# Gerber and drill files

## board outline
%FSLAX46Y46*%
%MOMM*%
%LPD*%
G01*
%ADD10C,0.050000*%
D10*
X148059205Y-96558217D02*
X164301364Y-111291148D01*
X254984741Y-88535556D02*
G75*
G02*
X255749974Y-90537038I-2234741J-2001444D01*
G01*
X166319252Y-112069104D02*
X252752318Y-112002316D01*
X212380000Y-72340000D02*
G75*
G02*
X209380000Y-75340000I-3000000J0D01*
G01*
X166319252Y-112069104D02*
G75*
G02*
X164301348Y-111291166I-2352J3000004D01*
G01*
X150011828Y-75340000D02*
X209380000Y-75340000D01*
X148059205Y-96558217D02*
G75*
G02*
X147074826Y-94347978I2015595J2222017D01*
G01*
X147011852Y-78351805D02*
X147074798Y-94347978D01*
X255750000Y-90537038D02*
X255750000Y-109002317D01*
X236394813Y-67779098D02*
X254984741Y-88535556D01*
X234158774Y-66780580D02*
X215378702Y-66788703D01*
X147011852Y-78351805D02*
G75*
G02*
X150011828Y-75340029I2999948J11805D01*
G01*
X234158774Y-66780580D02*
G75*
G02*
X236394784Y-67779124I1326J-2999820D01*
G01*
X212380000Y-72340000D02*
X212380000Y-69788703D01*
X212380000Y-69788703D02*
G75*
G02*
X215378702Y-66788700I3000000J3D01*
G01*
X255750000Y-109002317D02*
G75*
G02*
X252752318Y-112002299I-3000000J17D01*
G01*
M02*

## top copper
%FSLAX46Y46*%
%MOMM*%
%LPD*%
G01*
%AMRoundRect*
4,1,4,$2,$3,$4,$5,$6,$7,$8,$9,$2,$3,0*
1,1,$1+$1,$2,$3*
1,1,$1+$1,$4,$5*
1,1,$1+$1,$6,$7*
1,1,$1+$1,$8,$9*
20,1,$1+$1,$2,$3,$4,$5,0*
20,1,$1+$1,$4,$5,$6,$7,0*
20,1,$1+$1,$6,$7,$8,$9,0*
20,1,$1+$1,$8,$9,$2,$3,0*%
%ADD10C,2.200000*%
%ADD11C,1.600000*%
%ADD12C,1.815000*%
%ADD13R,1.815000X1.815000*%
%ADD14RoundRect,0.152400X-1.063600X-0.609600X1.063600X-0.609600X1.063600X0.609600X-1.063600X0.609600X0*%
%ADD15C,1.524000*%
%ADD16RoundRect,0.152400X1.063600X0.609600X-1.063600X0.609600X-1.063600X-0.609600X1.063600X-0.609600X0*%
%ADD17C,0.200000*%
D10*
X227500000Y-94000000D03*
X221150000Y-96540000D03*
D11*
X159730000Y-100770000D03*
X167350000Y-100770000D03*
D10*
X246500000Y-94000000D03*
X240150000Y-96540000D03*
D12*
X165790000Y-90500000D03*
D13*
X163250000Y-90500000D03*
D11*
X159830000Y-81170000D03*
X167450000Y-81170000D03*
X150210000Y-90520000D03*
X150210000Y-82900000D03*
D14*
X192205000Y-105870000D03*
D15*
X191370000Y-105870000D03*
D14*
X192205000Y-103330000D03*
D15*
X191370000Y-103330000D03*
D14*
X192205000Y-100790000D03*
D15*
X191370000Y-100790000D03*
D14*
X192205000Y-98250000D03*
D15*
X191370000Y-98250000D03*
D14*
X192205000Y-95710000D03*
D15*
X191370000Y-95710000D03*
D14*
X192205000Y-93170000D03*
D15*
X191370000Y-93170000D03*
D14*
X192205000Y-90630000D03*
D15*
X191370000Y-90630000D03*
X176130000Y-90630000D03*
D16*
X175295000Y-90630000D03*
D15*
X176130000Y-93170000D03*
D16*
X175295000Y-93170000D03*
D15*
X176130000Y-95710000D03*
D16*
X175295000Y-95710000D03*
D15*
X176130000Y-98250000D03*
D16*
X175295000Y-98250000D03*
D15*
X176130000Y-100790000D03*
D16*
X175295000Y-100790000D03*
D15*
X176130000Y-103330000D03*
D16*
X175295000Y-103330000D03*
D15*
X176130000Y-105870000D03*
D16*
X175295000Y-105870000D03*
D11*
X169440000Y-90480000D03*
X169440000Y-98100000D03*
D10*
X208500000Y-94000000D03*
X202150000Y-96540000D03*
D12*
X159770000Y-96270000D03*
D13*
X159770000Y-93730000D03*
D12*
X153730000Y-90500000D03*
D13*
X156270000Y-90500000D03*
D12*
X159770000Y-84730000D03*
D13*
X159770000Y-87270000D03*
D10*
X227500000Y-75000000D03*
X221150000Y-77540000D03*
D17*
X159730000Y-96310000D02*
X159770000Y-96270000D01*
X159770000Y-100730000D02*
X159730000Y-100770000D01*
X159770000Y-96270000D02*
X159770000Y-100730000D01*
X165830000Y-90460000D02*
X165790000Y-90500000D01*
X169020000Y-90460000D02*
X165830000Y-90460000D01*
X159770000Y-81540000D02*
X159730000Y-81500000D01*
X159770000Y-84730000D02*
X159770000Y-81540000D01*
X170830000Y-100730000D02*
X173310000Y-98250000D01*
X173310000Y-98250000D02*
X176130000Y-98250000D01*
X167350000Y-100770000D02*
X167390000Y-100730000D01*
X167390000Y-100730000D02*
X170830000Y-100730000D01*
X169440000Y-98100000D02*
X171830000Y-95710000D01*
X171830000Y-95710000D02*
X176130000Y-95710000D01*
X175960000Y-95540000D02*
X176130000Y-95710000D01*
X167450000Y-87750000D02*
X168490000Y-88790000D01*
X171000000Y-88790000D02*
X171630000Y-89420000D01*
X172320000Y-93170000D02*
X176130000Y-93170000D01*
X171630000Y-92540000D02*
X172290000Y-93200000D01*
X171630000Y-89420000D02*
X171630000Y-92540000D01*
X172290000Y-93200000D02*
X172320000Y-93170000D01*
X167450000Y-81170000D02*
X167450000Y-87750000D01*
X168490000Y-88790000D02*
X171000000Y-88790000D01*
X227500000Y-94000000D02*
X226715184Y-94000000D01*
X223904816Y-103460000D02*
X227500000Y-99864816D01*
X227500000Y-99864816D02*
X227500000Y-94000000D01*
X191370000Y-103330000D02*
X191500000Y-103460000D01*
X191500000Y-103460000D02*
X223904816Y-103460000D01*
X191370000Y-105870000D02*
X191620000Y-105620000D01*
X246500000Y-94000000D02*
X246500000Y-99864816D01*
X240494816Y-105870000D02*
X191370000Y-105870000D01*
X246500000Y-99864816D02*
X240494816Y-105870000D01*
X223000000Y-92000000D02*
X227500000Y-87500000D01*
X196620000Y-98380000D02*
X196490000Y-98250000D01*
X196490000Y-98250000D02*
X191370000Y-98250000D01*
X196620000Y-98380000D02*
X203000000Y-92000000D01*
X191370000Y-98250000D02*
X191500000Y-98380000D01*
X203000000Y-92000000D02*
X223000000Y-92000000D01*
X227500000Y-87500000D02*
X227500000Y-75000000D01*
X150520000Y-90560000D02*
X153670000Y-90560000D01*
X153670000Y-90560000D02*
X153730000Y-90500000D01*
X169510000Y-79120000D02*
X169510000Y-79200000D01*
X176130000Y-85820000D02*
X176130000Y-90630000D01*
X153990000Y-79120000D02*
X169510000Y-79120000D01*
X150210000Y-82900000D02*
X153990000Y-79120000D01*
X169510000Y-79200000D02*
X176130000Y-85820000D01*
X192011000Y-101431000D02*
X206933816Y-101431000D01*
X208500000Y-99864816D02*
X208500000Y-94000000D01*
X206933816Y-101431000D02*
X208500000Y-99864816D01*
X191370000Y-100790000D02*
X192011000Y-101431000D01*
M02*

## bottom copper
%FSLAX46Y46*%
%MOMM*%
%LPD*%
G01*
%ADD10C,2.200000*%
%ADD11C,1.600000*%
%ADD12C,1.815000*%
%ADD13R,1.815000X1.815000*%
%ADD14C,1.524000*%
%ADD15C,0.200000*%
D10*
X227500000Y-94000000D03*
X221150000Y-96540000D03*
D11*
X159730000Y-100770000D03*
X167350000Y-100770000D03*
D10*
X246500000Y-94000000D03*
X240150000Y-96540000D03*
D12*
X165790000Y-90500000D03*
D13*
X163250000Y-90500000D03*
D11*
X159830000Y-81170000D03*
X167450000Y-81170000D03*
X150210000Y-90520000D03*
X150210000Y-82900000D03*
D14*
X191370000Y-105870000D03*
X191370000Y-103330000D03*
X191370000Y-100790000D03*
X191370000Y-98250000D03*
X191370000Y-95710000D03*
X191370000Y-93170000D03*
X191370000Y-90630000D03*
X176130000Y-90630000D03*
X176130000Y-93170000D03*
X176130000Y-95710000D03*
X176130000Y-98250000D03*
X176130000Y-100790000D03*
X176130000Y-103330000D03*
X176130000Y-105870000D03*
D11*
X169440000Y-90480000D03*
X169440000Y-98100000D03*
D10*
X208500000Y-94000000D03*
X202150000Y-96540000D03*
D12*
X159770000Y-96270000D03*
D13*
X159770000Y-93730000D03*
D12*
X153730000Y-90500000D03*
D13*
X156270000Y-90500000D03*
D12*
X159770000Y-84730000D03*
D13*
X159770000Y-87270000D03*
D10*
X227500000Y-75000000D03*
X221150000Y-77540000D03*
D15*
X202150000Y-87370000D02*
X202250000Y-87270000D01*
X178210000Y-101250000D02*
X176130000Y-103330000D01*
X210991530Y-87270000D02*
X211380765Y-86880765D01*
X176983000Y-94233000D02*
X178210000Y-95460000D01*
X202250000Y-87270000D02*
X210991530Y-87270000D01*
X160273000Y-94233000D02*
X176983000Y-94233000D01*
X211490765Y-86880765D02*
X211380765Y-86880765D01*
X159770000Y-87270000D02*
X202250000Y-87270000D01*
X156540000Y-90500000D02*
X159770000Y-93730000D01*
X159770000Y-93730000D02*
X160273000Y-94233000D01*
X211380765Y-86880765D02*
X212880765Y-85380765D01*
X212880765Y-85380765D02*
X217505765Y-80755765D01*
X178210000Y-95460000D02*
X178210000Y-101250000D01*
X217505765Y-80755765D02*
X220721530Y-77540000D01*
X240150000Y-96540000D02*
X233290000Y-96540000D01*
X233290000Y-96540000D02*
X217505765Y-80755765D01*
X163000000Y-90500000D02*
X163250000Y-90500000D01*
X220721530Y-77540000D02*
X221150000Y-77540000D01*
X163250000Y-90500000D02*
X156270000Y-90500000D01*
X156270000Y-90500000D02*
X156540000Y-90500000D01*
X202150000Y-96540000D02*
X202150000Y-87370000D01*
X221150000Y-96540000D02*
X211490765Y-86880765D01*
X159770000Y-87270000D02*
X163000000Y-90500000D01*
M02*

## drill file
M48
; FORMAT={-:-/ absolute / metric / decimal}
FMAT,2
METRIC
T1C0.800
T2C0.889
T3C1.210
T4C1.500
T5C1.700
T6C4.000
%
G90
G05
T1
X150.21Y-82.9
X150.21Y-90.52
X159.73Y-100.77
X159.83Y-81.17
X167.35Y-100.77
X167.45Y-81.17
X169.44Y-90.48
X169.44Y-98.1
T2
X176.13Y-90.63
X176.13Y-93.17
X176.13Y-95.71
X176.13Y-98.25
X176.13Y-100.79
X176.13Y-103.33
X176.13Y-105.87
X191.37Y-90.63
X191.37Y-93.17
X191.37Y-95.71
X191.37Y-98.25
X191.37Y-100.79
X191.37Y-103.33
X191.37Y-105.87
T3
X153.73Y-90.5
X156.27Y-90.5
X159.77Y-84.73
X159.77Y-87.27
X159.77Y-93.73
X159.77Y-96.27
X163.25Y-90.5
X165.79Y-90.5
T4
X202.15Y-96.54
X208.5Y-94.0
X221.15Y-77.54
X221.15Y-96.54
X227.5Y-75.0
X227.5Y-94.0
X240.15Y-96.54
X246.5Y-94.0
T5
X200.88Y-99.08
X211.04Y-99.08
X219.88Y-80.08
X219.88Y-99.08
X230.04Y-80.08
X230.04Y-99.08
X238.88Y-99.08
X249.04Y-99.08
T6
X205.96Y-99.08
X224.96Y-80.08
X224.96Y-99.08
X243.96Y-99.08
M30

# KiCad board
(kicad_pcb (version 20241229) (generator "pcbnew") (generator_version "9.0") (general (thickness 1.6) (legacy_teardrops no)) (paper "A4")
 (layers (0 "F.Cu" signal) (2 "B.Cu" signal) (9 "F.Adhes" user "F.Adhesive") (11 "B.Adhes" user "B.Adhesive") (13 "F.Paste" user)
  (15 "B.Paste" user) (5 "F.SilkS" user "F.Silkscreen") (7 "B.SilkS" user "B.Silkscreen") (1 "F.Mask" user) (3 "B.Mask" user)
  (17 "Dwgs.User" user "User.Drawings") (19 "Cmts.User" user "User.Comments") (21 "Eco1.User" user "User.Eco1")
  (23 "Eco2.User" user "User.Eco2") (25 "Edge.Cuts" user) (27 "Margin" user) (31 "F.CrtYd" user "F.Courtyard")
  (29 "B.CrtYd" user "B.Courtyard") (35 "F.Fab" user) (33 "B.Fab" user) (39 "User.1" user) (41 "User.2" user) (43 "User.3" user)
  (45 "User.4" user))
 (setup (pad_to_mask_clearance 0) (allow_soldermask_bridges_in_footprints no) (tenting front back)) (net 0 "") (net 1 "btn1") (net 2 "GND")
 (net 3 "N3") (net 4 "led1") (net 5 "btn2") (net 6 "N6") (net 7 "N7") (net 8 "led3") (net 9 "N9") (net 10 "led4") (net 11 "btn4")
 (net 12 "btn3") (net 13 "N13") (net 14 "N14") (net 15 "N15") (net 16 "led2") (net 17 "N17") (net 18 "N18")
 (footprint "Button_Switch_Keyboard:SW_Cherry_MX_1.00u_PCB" (layer "F.Cu") (at 227.5 94)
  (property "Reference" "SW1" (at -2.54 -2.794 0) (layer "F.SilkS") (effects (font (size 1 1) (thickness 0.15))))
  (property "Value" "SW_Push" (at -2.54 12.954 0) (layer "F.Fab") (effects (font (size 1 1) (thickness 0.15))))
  (pad "" np_thru_hole circle (at -7.62 5.08) (size 1.7 1.7) (drill 1.7) (layers "*.Cu" "*.Mask"))
  (pad "" np_thru_hole circle (at -2.54 5.08) (size 4 4) (drill 4) (layers "*.Cu" "*.Mask"))
  (pad "" np_thru_hole circle (at 2.54 5.08) (size 1.7 1.7) (drill 1.7) (layers "*.Cu" "*.Mask"))
  (pad "1" thru_hole circle (at 0 0) (size 2.2 2.2) (drill 1.5) (layers "*.Cu" "*.Mask") (remove_unused_layers no) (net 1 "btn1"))
  (pad "2" thru_hole circle (at -6.35 2.54) (size 2.2 2.2) (drill 1.5) (layers "*.Cu" "*.Mask") (remove_unused_layers no) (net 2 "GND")))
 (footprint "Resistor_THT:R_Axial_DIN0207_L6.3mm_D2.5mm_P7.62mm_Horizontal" (layer "F.Cu") (at 159.73 100.77)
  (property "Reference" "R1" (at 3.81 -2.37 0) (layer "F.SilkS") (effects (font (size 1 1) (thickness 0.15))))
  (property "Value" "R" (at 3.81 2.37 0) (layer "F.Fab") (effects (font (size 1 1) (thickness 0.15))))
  (pad "1" thru_hole circle (at 0 0) (size 1.6 1.6) (drill 0.8) (layers "*.Cu" "*.Mask") (remove_unused_layers no) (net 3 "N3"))
  (pad "2" thru_hole circle (at 7.62 0) (size 1.6 1.6) (drill 0.8) (layers "*.Cu" "*.Mask") (remove_unused_layers no) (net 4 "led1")))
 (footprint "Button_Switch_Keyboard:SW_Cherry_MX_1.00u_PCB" (layer "F.Cu") (at 246.5 94)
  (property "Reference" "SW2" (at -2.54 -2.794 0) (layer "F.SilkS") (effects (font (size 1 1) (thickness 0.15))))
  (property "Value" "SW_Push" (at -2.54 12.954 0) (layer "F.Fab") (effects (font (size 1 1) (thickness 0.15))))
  (pad "" np_thru_hole circle (at -7.62 5.08) (size 1.7 1.7) (drill 1.7) (layers "*.Cu" "*.Mask"))
  (pad "" np_thru_hole circle (at -2.54 5.08) (size 4 4) (drill 4) (layers "*.Cu" "*.Mask"))
  (pad "" np_thru_hole circle (at 2.54 5.08) (size 1.7 1.7) (drill 1.7) (layers "*.Cu" "*.Mask"))
  (pad "1" thru_hole circle (at 0 0) (size 2.2 2.2) (drill 1.5) (layers "*.Cu" "*.Mask") (remove_unused_layers no) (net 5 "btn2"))
  (pad "2" thru_hole circle (at -6.35 2.54) (size 2.2 2.2) (drill 1.5) (layers "*.Cu" "*.Mask") (remove_unused_layers no) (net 2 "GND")))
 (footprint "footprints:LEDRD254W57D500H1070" (layer "F.Cu") (at 164.52 90.5)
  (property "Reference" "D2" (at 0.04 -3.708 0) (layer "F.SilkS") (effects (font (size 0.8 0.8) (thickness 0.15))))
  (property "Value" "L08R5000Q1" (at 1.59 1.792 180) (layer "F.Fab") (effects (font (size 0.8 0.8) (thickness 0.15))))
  (pad "A" thru_hole circle (at 1.27 0) (size 1.815 1.815) (drill 1.21) (layers "*.Cu" "*.Mask") (remove_unused_layers no) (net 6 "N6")
   (solder_mask_margin 0.102))
  (pad "C" thru_hole rect (at -1.27 0) (size 1.815 1.815) (drill 1.21) (layers "*.Cu" "*.Mask") (remove_unused_layers no) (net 2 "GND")
   (solder_mask_margin 0.102)))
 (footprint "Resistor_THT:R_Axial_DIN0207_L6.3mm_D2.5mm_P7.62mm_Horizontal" (layer "F.Cu") (at 159.83 81.17)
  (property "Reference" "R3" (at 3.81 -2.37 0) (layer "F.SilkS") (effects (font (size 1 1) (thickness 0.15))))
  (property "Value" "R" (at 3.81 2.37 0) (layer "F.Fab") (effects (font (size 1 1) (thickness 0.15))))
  (pad "1" thru_hole circle (at 0 0) (size 1.6 1.6) (drill 0.8) (layers "*.Cu" "*.Mask") (remove_unused_layers no) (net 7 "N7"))
  (pad "2" thru_hole circle (at 7.62 0) (size 1.6 1.6) (drill 0.8) (layers "*.Cu" "*.Mask") (remove_unused_layers no) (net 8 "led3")))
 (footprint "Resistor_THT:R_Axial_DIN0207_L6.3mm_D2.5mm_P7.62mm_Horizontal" (layer "F.Cu") (at 150.21 90.52 90)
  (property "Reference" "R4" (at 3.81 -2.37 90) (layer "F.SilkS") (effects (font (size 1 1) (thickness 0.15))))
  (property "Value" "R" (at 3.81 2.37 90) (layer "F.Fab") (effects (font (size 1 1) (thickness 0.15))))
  (pad "1" thru_hole circle (at 0 0 90) (size 1.6 1.6) (drill 0.8) (layers "*.Cu" "*.Mask") (remove_unused_layers no) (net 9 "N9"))
  (pad "2" thru_hole circle (at 7.62 0 90) (size 1.6 1.6) (drill 0.8) (layers "*.Cu" "*.Mask") (remove_unused_layers no) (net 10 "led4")))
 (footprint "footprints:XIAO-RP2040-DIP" (layer "F.Cu") (at 183.75 98.25 -90)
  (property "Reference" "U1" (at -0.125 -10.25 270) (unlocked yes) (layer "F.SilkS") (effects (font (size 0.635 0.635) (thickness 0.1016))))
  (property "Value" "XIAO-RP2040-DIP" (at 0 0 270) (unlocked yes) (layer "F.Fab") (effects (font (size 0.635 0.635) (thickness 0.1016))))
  (pad "1" smd roundrect (at 7.62 -8.455) (size 2.432 1.524) (layers "F.Cu" "F.Mask") (roundrect_rratio 0.1) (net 5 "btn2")
   (thermal_bridge_angle 45))
  (pad "1" thru_hole circle (at 7.62 -7.62) (size 1.524 1.524) (drill 0.889) (layers "*.Cu" "*.Mask") (remove_unused_layers no)
   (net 5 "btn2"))
  (pad "2" smd roundrect (at 5.08 -8.455) (size 2.432 1.524) (layers "F.Cu" "F.Mask") (roundrect_rratio 0.1) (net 1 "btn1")
   (thermal_bridge_angle 45))
  (pad "2" thru_hole circle (at 5.08 -7.62) (size 1.524 1.524) (drill 0.889) (layers "*.Cu" "*.Mask") (remove_unused_layers no)
   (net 1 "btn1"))
  (pad "3" smd roundrect (at 2.54 -8.455) (size 2.432 1.524) (layers "F.Cu" "F.Mask") (roundrect_rratio 0.1) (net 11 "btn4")
   (thermal_bridge_angle 45))
  (pad "3" thru_hole circle (at 2.54 -7.62) (size 1.524 1.524) (drill 0.889) (layers "*.Cu" "*.Mask") (remove_unused_layers no)
   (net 11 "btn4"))
  (pad "4" smd roundrect (at 0 -8.455) (size 2.432 1.524) (layers "F.Cu" "F.Mask") (roundrect_rratio 0.1) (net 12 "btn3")
   (thermal_bridge_angle 45))
  (pad "4" thru_hole circle (at 0 -7.62) (size 1.524 1.524) (drill 0.889) (layers "*.Cu" "*.Mask") (remove_unused_layers no) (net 12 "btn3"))
  (pad "5" smd roundrect (at -2.54 -8.455) (size 2.432 1.524) (layers "F.Cu" "F.Mask") (roundrect_rratio 0.1) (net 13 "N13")
   (thermal_bridge_angle 45))
  (pad "5" thru_hole circle (at -2.54 -7.62) (size 1.524 1.524) (drill 0.889) (layers "*.Cu" "*.Mask") (remove_unused_layers no)
   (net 13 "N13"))
  (pad "6" smd roundrect (at -5.08 -8.455) (size 2.432 1.524) (layers "F.Cu" "F.Mask") (roundrect_rratio 0.1) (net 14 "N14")
   (thermal_bridge_angle 45))
  (pad "6" thru_hole circle (at -5.08 -7.62) (size 1.524 1.524) (drill 0.889) (layers "*.Cu" "*.Mask") (remove_unused_layers no)
   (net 14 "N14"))
  (pad "7" smd roundrect (at -7.62 -8.455) (size 2.432 1.524) (layers "F.Cu" "F.Mask") (roundrect_rratio 0.1) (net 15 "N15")
   (thermal_bridge_angle 45))
  (pad "7" thru_hole circle (at -7.62 -7.62) (size 1.524 1.524) (drill 0.889) (layers "*.Cu" "*.Mask") (remove_unused_layers no)
   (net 15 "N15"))
  (pad "8" thru_hole circle (at -7.62 7.62 180) (size 1.524 1.524) (drill 0.889) (layers "*.Cu" "*.Mask") (remove_unused_layers no)
   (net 10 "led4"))
  (pad "8" smd roundrect (at -7.62 8.455 180) (size 2.432 1.524) (layers "F.Cu" "F.Mask") (roundrect_rratio 0.1) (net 10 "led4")
   (thermal_bridge_angle 45))
  (pad "9" thru_hole circle (at -5.08 7.62 180) (size 1.524 1.524) (drill 0.889) (layers "*.Cu" "*.Mask") (remove_unused_layers no)
   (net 8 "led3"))
  (pad "9" smd roundrect (at -5.08 8.455 180) (size 2.432 1.524) (layers "F.Cu" "F.Mask") (roundrect_rratio 0.1) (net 8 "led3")
   (thermal_bridge_angle 45))
  (pad "10" thru_hole circle (at -2.54 7.62 180) (size 1.524 1.524) (drill 0.889) (layers "*.Cu" "*.Mask") (remove_unused_layers no)
   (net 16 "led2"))
  (pad "10" smd roundrect (at -2.54 8.455 180) (size 2.432 1.524) (layers "F.Cu" "F.Mask") (roundrect_rratio 0.1) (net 16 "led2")
   (thermal_bridge_angle 45))
  (pad "11" thru_hole circle (at 0 7.62 180) (size 1.524 1.524) (drill 0.889) (layers "*.Cu" "*.Mask") (remove_unused_layers no)
   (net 4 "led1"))
  (pad "11" smd roundrect (at 0 8.455 180) (size 2.432 1.524) (layers "F.Cu" "F.Mask") (roundrect_rratio 0.1) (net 4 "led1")
   (thermal_bridge_angle 45))
  (pad "12" thru_hole circle (at 2.54 7.62 180) (size 1.524 1.524) (drill 0.889) (layers "*.Cu" "*.Mask") (remove_unused_layers no)
   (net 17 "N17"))
  (pad "12" smd roundrect (at 2.54 8.455 180) (size 2.432 1.524) (layers "F.Cu" "F.Mask") (roundrect_rratio 0.1) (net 17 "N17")
   (thermal_bridge_angle 45))
  (pad "13" thru_hole circle (at 5.08 7.62 180) (size 1.524 1.524) (drill 0.889) (layers "*.Cu" "*.Mask") (remove_unused_layers no)
   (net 2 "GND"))
  (pad "13" smd roundrect (at 5.08 8.455 180) (size 2.432 1.524) (layers "F.Cu" "F.Mask") (roundrect_rratio 0.1) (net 2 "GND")
   (thermal_bridge_angle 45))
  (pad "14" thru_hole circle (at 7.62 7.62 180) (size 1.524 1.524) (drill 0.889) (layers "*.Cu" "*.Mask") (remove_unused_layers no)
   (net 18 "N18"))
  (pad "14" smd roundrect (at 7.62 8.455 180) (size 2.432 1.524) (layers "F.Cu" "F.Mask") (roundrect_rratio 0.1) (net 18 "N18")
   (thermal_bridge_angle 45)))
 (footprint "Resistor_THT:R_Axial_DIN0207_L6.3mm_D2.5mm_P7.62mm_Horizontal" (layer "F.Cu") (at 169.44 90.48 -90)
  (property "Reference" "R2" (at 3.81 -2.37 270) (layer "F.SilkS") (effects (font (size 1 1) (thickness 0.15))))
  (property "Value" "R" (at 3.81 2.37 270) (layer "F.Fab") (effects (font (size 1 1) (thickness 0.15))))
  (pad "1" thru_hole circle (at 0 0 270) (size 1.6 1.6) (drill 0.8) (layers "*.Cu" "*.Mask") (remove_unused_layers no) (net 6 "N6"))
  (pad "2" thru_hole circle (at 7.62 0 270) (size 1.6 1.6) (drill 0.8) (layers "*.Cu" "*.Mask") (remove_unused_layers no) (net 16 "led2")))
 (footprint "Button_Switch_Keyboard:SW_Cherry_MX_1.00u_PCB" (layer "F.Cu") (at 208.5 94)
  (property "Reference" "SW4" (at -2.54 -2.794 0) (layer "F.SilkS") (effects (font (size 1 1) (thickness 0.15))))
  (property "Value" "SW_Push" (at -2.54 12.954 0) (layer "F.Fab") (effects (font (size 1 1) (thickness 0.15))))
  (pad "" np_thru_hole circle (at -7.62 5.08) (size 1.7 1.7) (drill 1.7) (layers "*.Cu" "*.Mask"))
  (pad "" np_thru_hole circle (at -2.54 5.08) (size 4 4) (drill 4) (layers "*.Cu" "*.Mask"))
  (pad "" np_thru_hole circle (at 2.54 5.08) (size 1.7 1.7) (drill 1.7) (layers "*.Cu" "*.Mask"))
  (pad "1" thru_hole circle (at 0 0) (size 2.2 2.2) (drill 1.5) (layers "*.Cu" "*.Mask") (remove_unused_layers no) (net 11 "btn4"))
  (pad "2" thru_hole circle (at -6.35 2.54) (size 2.2 2.2) (drill 1.5) (layers "*.Cu" "*.Mask") (remove_unused_layers no) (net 2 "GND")))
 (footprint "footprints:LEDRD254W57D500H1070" (layer "F.Cu") (at 159.77 95 -90)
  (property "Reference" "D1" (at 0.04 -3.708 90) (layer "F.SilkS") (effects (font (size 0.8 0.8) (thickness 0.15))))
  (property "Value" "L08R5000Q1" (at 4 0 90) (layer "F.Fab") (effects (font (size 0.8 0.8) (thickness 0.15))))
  (pad "A" thru_hole circle (at 1.27 0 270) (size 1.815 1.815) (drill 1.21) (layers "*.Cu" "*.Mask") (remove_unused_layers no) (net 3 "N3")
   (solder_mask_margin 0.102))
  (pad "C" thru_hole rect (at -1.27 0 270) (size 1.815 1.815) (drill 1.21) (layers "*.Cu" "*.Mask") (remove_unused_layers no) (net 2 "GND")
   (solder_mask_margin 0.102)))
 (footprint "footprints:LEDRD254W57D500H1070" (layer "F.Cu") (at 155 90.5 180)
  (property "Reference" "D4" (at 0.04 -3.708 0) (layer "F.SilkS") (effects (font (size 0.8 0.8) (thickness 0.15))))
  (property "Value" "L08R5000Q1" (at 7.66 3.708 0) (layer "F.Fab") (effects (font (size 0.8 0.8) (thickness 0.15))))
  (pad "A" thru_hole circle (at 1.27 0 180) (size 1.815 1.815) (drill 1.21) (layers "*.Cu" "*.Mask") (remove_unused_layers no) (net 9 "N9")
   (solder_mask_margin 0.102))
  (pad "C" thru_hole rect (at -1.27 0 180) (size 1.815 1.815) (drill 1.21) (layers "*.Cu" "*.Mask") (remove_unused_layers no) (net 2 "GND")
   (solder_mask_margin 0.102)))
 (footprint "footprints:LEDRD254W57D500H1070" (layer "F.Cu") (at 159.77 86 90)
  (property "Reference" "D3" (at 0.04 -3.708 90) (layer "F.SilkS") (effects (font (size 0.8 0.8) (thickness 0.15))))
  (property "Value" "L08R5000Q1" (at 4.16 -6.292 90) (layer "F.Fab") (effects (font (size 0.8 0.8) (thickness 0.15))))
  (pad "A" thru_hole circle (at 1.27 0 90) (size 1.815 1.815) (drill 1.21) (layers "*.Cu" "*.Mask") (remove_unused_layers no) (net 7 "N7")
   (solder_mask_margin 0.102))
  (pad "C" thru_hole rect (at -1.27 0 90) (size 1.815 1.815) (drill 1.21) (layers "*.Cu" "*.Mask") (remove_unused_layers no) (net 2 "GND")
   (solder_mask_margin 0.102)))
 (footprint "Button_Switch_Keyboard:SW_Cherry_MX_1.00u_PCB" (layer "F.Cu") (at 227.5 75)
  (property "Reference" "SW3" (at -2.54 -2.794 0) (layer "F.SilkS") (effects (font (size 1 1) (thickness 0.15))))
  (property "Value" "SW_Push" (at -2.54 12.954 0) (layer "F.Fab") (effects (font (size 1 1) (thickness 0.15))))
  (pad "" np_thru_hole circle (at -7.62 5.08) (size 1.7 1.7) (drill 1.7) (layers "*.Cu" "*.Mask"))
  (pad "" np_thru_hole circle (at -2.54 5.08) (size 4 4) (drill 4) (layers "*.Cu" "*.Mask"))
  (pad "" np_thru_hole circle (at 2.54 5.08) (size 1.7 1.7) (drill 1.7) (layers "*.Cu" "*.Mask"))
  (pad "1" thru_hole circle (at 0 0) (size 2.2 2.2) (drill 1.5) (layers "*.Cu" "*.Mask") (remove_unused_layers no) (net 12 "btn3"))
  (pad "2" thru_hole circle (at -6.35 2.54) (size 2.2 2.2) (drill 1.5) (layers "*.Cu" "*.Mask") (remove_unused_layers no) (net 2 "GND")))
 (gr_line (start 148.059205 96.558217) (end 164.301364 111.291148) (stroke (width 0.05) (type default)) (layer "Edge.Cuts"))
 (gr_arc (start 254.984741 88.535556) (mid 255.552162 89.465643) (end 255.75 90.537038) (stroke (width 0.05) (type default))
  (layer "Edge.Cuts"))
 (gr_line (start 166.319252 112.069104) (end 252.752318 112.002316) (stroke (width 0.05) (type default)) (layer "Edge.Cuts"))
 (gr_arc (start 212.38 72.34) (mid 211.50132 74.46132) (end 209.38 75.34) (stroke (width 0.05) (type default)) (layer "Edge.Cuts"))
 (gr_arc (start 166.319252 112.069104) (mid 165.237768 111.868283) (end 164.301364 111.291148) (stroke (width 0.05) (type default))
  (layer "Edge.Cuts"))
 (gr_line (start 150.011828 75.34) (end 209.38 75.34) (stroke (width 0.05) (type default)) (layer "Edge.Cuts"))
 (gr_arc (start 148.059205 96.558217) (mid 147.334297 95.55674) (end 147.074798 94.347978) (stroke (width 0.05) (type default))
  (layer "Edge.Cuts"))
 (gr_line (start 147.011852 78.351805) (end 147.074798 94.347978) (stroke (width 0.05) (type default)) (layer "Edge.Cuts"))
 (gr_line (start 255.75 90.537038) (end 255.75 109.002317) (stroke (width 0.05) (type default)) (layer "Edge.Cuts"))
 (gr_line (start 236.394813 67.779098) (end 254.984741 88.535556) (stroke (width 0.05) (type default)) (layer "Edge.Cuts"))
 (gr_line (start 234.158774 66.78058) (end 215.378702 66.788703) (stroke (width 0.05) (type default)) (layer "Edge.Cuts"))
 (gr_arc (start 147.011852 78.351805) (mid 147.88634 76.222868) (end 150.011828 75.34) (stroke (width 0.05) (type default))
  (layer "Edge.Cuts"))
 (gr_arc (start 234.158774 66.78058) (mid 235.383324 67.041286) (end 236.394813 67.779098) (stroke (width 0.05) (type default))
  (layer "Edge.Cuts"))
 (gr_line (start 212.38 72.34) (end 212.38 69.788703) (stroke (width 0.05) (type default)) (layer "Edge.Cuts"))
 (gr_arc (start 212.38 69.788703) (mid 213.258221 67.667842) (end 215.378702 66.788703) (stroke (width 0.05) (type default))
  (layer "Edge.Cuts"))
 (gr_arc (start 255.75 109.002317) (mid 254.872134 111.122807) (end 252.752318 112.002316) (stroke (width 0.05) (type default))
  (layer "Edge.Cuts"))
 (segment (start 202.15 87.37) (end 202.25 87.27) (width 0.2) (layer "B.Cu") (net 2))
 (segment (start 178.21 101.25) (end 176.13 103.33) (width 0.2) (layer "B.Cu") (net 2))
 (segment (start 210.99153 87.27) (end 211.380765 86.880765) (width 0.2) (layer "B.Cu") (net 2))
 (segment (start 176.983 94.233) (end 178.21 95.46) (width 0.2) (layer "B.Cu") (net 2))
 (segment (start 202.25 87.27) (end 210.99153 87.27) (width 0.2) (layer "B.Cu") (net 2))
 (segment (start 160.273 94.233) (end 176.983 94.233) (width 0.2) (layer "B.Cu") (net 2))
 (segment (start 211.490765 86.880765) (end 211.380765 86.880765) (width 0.2) (layer "B.Cu") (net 2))
 (segment (start 159.77 87.27) (end 202.25 87.27) (width 0.2) (layer "B.Cu") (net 2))
 (segment (start 156.54 90.5) (end 159.77 93.73) (width 0.2) (layer "B.Cu") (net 2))
 (segment (start 159.77 93.73) (end 160.273 94.233) (width 0.2) (layer "B.Cu") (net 2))
 (segment (start 211.380765 86.880765) (end 212.880765 85.380765) (width 0.2) (layer "B.Cu") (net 2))
 (segment (start 212.880765 85.380765) (end 217.505765 80.755765) (width 0.2) (layer "B.Cu") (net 2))
 (segment (start 178.21 95.46) (end 178.21 101.25) (width 0.2) (layer "B.Cu") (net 2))
 (segment (start 217.505765 80.755765) (end 220.72153 77.54) (width 0.2) (layer "B.Cu") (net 2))
 (segment (start 240.15 96.54) (end 233.29 96.54) (width 0.2) (layer "B.Cu") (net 2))
 (segment (start 233.29 96.54) (end 217.505765 80.755765) (width 0.2) (layer "B.Cu") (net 2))
 (segment (start 163 90.5) (end 163.25 90.5) (width 0.2) (layer "B.Cu") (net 2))
 (segment (start 220.72153 77.54) (end 221.15 77.54) (width 0.2) (layer "B.Cu") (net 2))
 (segment (start 163.25 90.5) (end 156.27 90.5) (width 0.2) (layer "B.Cu") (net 2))
 (segment (start 156.27 90.5) (end 156.54 90.5) (width 0.2) (layer "B.Cu") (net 2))
 (segment (start 202.15 96.54) (end 202.15 87.37) (width 0.2) (layer "B.Cu") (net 2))
 (segment (start 221.15 96.54) (end 211.490765 86.880765) (width 0.2) (layer "B.Cu") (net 2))
 (segment (start 159.77 87.27) (end 163 90.5) (width 0.2) (layer "B.Cu") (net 2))
 (segment (start 159.73 96.31) (end 159.77 96.27) (width 0.2) (layer "F.Cu") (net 3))
 (segment (start 159.77 100.73) (end 159.73 100.77) (width 0.2) (layer "F.Cu") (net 3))
 (segment (start 159.77 96.27) (end 159.77 100.73) (width 0.2) (layer "F.Cu") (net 3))
 (segment (start 165.83 90.46) (end 165.79 90.5) (width 0.2) (layer "F.Cu") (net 6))
 (segment (start 169.02 90.46) (end 165.83 90.46) (width 0.2) (layer "F.Cu") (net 6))
 (segment (start 159.77 81.54) (end 159.73 81.5) (width 0.2) (layer "F.Cu") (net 7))
 (segment (start 159.77 84.73) (end 159.77 81.54) (width 0.2) (layer "F.Cu") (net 7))
 (segment (start 170.83 100.73) (end 173.31 98.25) (width 0.2) (layer "F.Cu") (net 4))
 (segment (start 173.31 98.25) (end 176.13 98.25) (width 0.2) (layer "F.Cu") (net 4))
 (segment (start 167.35 100.77) (end 167.39 100.73) (width 0.2) (layer "F.Cu") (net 4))
 (segment (start 167.39 100.73) (end 170.83 100.73) (width 0.2) (layer "F.Cu") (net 4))
 (segment (start 169.44 98.1) (end 171.83 95.71) (width 0.2) (layer "F.Cu") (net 16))
 (segment (start 171.83 95.71) (end 176.13 95.71) (width 0.2) (layer "F.Cu") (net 16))
 (segment (start 175.96 95.54) (end 176.13 95.71) (width 0.2) (layer "F.Cu") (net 16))
 (segment (start 167.45 87.75) (end 168.49 88.79) (width 0.2) (layer "F.Cu") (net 8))
 (segment (start 171 88.79) (end 171.63 89.42) (width 0.2) (layer "F.Cu") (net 8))
 (segment (start 172.32 93.17) (end 176.13 93.17) (width 0.2) (layer "F.Cu") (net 8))
 (segment (start 171.63 92.54) (end 172.29 93.2) (width 0.2) (layer "F.Cu") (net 8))
 (segment (start 171.63 89.42) (end 171.63 92.54) (width 0.2) (layer "F.Cu") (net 8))
 (segment (start 172.29 93.2) (end 172.32 93.17) (width 0.2) (layer "F.Cu") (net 8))
 (segment (start 167.45 81.17) (end 167.45 87.75) (width 0.2) (layer "F.Cu") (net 8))
 (segment (start 168.49 88.79) (end 171 88.79) (width 0.2) (layer "F.Cu") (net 8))
 (segment (start 227.5 94) (end 226.715184 94) (width 0.2) (layer "F.Cu") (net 1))
 (segment (start 223.904816 103.46) (end 227.5 99.864816) (width 0.2) (layer "F.Cu") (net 1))
 (segment (start 227.5 99.864816) (end 227.5 94) (width 0.2) (layer "F.Cu") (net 1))
 (segment (start 191.37 103.33) (end 191.5 103.46) (width 0.2) (layer "F.Cu") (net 1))
 (segment (start 191.5 103.46) (end 223.904816 103.46) (width 0.2) (layer "F.Cu") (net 1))
 (segment (start 191.37 105.87) (end 191.62 105.62) (width 0.2) (layer "F.Cu") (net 5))
 (segment (start 246.5 94) (end 246.5 99.864816) (width 0.2) (layer "F.Cu") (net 5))
 (segment (start 240.494816 105.87) (end 191.37 105.87) (width 0.2) (layer "F.Cu") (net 5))
 (segment (start 246.5 99.864816) (end 240.494816 105.87) (width 0.2) (layer "F.Cu") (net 5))
 (segment (start 223 92) (end 227.5 87.5) (width 0.2) (layer "F.Cu") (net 12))
 (segment (start 196.62 98.38) (end 196.49 98.25) (width 0.2) (layer "F.Cu") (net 12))
 (segment (start 196.49 98.25) (end 191.37 98.25) (width 0.2) (layer "F.Cu") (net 12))
 (segment (start 196.62 98.38) (end 203 92) (width 0.2) (layer "F.Cu") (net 12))
 (segment (start 191.37 98.25) (end 191.5 98.38) (width 0.2) (layer "F.Cu") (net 12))
 (segment (start 203 92) (end 223 92) (width 0.2) (layer "F.Cu") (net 12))
 (segment (start 227.5 87.5) (end 227.5 75) (width 0.2) (layer "F.Cu") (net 12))
 (segment (start 150.52 90.56) (end 153.67 90.56) (width 0.2) (layer "F.Cu") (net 9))
 (segment (start 153.67 90.56) (end 153.73 90.5) (width 0.2) (layer "F.Cu") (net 9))
 (segment (start 169.51 79.12) (end 169.51 79.2) (width 0.2) (layer "F.Cu") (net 10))
 (segment (start 176.13 85.82) (end 176.13 90.63) (width 0.2) (layer "F.Cu") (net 10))
 (segment (start 153.99 79.12) (end 169.51 79.12) (width 0.2) (layer "F.Cu") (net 10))
 (segment (start 150.21 82.9) (end 153.99 79.12) (width 0.2) (layer "F.Cu") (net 10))
 (segment (start 169.51 79.2) (end 176.13 85.82) (width 0.2) (layer "F.Cu") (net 10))
 (segment (start 192.011 101.431) (end 206.933816 101.431) (width 0.2) (layer "F.Cu") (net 11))
 (segment (start 208.5 99.864816) (end 208.5 94) (width 0.2) (layer "F.Cu") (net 11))
 (segment (start 206.933816 101.431) (end 208.5 99.864816) (width 0.2) (layer "F.Cu") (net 11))
 (segment (start 191.37 100.79) (end 192.011 101.431) (width 0.2) (layer "F.Cu") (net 11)))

